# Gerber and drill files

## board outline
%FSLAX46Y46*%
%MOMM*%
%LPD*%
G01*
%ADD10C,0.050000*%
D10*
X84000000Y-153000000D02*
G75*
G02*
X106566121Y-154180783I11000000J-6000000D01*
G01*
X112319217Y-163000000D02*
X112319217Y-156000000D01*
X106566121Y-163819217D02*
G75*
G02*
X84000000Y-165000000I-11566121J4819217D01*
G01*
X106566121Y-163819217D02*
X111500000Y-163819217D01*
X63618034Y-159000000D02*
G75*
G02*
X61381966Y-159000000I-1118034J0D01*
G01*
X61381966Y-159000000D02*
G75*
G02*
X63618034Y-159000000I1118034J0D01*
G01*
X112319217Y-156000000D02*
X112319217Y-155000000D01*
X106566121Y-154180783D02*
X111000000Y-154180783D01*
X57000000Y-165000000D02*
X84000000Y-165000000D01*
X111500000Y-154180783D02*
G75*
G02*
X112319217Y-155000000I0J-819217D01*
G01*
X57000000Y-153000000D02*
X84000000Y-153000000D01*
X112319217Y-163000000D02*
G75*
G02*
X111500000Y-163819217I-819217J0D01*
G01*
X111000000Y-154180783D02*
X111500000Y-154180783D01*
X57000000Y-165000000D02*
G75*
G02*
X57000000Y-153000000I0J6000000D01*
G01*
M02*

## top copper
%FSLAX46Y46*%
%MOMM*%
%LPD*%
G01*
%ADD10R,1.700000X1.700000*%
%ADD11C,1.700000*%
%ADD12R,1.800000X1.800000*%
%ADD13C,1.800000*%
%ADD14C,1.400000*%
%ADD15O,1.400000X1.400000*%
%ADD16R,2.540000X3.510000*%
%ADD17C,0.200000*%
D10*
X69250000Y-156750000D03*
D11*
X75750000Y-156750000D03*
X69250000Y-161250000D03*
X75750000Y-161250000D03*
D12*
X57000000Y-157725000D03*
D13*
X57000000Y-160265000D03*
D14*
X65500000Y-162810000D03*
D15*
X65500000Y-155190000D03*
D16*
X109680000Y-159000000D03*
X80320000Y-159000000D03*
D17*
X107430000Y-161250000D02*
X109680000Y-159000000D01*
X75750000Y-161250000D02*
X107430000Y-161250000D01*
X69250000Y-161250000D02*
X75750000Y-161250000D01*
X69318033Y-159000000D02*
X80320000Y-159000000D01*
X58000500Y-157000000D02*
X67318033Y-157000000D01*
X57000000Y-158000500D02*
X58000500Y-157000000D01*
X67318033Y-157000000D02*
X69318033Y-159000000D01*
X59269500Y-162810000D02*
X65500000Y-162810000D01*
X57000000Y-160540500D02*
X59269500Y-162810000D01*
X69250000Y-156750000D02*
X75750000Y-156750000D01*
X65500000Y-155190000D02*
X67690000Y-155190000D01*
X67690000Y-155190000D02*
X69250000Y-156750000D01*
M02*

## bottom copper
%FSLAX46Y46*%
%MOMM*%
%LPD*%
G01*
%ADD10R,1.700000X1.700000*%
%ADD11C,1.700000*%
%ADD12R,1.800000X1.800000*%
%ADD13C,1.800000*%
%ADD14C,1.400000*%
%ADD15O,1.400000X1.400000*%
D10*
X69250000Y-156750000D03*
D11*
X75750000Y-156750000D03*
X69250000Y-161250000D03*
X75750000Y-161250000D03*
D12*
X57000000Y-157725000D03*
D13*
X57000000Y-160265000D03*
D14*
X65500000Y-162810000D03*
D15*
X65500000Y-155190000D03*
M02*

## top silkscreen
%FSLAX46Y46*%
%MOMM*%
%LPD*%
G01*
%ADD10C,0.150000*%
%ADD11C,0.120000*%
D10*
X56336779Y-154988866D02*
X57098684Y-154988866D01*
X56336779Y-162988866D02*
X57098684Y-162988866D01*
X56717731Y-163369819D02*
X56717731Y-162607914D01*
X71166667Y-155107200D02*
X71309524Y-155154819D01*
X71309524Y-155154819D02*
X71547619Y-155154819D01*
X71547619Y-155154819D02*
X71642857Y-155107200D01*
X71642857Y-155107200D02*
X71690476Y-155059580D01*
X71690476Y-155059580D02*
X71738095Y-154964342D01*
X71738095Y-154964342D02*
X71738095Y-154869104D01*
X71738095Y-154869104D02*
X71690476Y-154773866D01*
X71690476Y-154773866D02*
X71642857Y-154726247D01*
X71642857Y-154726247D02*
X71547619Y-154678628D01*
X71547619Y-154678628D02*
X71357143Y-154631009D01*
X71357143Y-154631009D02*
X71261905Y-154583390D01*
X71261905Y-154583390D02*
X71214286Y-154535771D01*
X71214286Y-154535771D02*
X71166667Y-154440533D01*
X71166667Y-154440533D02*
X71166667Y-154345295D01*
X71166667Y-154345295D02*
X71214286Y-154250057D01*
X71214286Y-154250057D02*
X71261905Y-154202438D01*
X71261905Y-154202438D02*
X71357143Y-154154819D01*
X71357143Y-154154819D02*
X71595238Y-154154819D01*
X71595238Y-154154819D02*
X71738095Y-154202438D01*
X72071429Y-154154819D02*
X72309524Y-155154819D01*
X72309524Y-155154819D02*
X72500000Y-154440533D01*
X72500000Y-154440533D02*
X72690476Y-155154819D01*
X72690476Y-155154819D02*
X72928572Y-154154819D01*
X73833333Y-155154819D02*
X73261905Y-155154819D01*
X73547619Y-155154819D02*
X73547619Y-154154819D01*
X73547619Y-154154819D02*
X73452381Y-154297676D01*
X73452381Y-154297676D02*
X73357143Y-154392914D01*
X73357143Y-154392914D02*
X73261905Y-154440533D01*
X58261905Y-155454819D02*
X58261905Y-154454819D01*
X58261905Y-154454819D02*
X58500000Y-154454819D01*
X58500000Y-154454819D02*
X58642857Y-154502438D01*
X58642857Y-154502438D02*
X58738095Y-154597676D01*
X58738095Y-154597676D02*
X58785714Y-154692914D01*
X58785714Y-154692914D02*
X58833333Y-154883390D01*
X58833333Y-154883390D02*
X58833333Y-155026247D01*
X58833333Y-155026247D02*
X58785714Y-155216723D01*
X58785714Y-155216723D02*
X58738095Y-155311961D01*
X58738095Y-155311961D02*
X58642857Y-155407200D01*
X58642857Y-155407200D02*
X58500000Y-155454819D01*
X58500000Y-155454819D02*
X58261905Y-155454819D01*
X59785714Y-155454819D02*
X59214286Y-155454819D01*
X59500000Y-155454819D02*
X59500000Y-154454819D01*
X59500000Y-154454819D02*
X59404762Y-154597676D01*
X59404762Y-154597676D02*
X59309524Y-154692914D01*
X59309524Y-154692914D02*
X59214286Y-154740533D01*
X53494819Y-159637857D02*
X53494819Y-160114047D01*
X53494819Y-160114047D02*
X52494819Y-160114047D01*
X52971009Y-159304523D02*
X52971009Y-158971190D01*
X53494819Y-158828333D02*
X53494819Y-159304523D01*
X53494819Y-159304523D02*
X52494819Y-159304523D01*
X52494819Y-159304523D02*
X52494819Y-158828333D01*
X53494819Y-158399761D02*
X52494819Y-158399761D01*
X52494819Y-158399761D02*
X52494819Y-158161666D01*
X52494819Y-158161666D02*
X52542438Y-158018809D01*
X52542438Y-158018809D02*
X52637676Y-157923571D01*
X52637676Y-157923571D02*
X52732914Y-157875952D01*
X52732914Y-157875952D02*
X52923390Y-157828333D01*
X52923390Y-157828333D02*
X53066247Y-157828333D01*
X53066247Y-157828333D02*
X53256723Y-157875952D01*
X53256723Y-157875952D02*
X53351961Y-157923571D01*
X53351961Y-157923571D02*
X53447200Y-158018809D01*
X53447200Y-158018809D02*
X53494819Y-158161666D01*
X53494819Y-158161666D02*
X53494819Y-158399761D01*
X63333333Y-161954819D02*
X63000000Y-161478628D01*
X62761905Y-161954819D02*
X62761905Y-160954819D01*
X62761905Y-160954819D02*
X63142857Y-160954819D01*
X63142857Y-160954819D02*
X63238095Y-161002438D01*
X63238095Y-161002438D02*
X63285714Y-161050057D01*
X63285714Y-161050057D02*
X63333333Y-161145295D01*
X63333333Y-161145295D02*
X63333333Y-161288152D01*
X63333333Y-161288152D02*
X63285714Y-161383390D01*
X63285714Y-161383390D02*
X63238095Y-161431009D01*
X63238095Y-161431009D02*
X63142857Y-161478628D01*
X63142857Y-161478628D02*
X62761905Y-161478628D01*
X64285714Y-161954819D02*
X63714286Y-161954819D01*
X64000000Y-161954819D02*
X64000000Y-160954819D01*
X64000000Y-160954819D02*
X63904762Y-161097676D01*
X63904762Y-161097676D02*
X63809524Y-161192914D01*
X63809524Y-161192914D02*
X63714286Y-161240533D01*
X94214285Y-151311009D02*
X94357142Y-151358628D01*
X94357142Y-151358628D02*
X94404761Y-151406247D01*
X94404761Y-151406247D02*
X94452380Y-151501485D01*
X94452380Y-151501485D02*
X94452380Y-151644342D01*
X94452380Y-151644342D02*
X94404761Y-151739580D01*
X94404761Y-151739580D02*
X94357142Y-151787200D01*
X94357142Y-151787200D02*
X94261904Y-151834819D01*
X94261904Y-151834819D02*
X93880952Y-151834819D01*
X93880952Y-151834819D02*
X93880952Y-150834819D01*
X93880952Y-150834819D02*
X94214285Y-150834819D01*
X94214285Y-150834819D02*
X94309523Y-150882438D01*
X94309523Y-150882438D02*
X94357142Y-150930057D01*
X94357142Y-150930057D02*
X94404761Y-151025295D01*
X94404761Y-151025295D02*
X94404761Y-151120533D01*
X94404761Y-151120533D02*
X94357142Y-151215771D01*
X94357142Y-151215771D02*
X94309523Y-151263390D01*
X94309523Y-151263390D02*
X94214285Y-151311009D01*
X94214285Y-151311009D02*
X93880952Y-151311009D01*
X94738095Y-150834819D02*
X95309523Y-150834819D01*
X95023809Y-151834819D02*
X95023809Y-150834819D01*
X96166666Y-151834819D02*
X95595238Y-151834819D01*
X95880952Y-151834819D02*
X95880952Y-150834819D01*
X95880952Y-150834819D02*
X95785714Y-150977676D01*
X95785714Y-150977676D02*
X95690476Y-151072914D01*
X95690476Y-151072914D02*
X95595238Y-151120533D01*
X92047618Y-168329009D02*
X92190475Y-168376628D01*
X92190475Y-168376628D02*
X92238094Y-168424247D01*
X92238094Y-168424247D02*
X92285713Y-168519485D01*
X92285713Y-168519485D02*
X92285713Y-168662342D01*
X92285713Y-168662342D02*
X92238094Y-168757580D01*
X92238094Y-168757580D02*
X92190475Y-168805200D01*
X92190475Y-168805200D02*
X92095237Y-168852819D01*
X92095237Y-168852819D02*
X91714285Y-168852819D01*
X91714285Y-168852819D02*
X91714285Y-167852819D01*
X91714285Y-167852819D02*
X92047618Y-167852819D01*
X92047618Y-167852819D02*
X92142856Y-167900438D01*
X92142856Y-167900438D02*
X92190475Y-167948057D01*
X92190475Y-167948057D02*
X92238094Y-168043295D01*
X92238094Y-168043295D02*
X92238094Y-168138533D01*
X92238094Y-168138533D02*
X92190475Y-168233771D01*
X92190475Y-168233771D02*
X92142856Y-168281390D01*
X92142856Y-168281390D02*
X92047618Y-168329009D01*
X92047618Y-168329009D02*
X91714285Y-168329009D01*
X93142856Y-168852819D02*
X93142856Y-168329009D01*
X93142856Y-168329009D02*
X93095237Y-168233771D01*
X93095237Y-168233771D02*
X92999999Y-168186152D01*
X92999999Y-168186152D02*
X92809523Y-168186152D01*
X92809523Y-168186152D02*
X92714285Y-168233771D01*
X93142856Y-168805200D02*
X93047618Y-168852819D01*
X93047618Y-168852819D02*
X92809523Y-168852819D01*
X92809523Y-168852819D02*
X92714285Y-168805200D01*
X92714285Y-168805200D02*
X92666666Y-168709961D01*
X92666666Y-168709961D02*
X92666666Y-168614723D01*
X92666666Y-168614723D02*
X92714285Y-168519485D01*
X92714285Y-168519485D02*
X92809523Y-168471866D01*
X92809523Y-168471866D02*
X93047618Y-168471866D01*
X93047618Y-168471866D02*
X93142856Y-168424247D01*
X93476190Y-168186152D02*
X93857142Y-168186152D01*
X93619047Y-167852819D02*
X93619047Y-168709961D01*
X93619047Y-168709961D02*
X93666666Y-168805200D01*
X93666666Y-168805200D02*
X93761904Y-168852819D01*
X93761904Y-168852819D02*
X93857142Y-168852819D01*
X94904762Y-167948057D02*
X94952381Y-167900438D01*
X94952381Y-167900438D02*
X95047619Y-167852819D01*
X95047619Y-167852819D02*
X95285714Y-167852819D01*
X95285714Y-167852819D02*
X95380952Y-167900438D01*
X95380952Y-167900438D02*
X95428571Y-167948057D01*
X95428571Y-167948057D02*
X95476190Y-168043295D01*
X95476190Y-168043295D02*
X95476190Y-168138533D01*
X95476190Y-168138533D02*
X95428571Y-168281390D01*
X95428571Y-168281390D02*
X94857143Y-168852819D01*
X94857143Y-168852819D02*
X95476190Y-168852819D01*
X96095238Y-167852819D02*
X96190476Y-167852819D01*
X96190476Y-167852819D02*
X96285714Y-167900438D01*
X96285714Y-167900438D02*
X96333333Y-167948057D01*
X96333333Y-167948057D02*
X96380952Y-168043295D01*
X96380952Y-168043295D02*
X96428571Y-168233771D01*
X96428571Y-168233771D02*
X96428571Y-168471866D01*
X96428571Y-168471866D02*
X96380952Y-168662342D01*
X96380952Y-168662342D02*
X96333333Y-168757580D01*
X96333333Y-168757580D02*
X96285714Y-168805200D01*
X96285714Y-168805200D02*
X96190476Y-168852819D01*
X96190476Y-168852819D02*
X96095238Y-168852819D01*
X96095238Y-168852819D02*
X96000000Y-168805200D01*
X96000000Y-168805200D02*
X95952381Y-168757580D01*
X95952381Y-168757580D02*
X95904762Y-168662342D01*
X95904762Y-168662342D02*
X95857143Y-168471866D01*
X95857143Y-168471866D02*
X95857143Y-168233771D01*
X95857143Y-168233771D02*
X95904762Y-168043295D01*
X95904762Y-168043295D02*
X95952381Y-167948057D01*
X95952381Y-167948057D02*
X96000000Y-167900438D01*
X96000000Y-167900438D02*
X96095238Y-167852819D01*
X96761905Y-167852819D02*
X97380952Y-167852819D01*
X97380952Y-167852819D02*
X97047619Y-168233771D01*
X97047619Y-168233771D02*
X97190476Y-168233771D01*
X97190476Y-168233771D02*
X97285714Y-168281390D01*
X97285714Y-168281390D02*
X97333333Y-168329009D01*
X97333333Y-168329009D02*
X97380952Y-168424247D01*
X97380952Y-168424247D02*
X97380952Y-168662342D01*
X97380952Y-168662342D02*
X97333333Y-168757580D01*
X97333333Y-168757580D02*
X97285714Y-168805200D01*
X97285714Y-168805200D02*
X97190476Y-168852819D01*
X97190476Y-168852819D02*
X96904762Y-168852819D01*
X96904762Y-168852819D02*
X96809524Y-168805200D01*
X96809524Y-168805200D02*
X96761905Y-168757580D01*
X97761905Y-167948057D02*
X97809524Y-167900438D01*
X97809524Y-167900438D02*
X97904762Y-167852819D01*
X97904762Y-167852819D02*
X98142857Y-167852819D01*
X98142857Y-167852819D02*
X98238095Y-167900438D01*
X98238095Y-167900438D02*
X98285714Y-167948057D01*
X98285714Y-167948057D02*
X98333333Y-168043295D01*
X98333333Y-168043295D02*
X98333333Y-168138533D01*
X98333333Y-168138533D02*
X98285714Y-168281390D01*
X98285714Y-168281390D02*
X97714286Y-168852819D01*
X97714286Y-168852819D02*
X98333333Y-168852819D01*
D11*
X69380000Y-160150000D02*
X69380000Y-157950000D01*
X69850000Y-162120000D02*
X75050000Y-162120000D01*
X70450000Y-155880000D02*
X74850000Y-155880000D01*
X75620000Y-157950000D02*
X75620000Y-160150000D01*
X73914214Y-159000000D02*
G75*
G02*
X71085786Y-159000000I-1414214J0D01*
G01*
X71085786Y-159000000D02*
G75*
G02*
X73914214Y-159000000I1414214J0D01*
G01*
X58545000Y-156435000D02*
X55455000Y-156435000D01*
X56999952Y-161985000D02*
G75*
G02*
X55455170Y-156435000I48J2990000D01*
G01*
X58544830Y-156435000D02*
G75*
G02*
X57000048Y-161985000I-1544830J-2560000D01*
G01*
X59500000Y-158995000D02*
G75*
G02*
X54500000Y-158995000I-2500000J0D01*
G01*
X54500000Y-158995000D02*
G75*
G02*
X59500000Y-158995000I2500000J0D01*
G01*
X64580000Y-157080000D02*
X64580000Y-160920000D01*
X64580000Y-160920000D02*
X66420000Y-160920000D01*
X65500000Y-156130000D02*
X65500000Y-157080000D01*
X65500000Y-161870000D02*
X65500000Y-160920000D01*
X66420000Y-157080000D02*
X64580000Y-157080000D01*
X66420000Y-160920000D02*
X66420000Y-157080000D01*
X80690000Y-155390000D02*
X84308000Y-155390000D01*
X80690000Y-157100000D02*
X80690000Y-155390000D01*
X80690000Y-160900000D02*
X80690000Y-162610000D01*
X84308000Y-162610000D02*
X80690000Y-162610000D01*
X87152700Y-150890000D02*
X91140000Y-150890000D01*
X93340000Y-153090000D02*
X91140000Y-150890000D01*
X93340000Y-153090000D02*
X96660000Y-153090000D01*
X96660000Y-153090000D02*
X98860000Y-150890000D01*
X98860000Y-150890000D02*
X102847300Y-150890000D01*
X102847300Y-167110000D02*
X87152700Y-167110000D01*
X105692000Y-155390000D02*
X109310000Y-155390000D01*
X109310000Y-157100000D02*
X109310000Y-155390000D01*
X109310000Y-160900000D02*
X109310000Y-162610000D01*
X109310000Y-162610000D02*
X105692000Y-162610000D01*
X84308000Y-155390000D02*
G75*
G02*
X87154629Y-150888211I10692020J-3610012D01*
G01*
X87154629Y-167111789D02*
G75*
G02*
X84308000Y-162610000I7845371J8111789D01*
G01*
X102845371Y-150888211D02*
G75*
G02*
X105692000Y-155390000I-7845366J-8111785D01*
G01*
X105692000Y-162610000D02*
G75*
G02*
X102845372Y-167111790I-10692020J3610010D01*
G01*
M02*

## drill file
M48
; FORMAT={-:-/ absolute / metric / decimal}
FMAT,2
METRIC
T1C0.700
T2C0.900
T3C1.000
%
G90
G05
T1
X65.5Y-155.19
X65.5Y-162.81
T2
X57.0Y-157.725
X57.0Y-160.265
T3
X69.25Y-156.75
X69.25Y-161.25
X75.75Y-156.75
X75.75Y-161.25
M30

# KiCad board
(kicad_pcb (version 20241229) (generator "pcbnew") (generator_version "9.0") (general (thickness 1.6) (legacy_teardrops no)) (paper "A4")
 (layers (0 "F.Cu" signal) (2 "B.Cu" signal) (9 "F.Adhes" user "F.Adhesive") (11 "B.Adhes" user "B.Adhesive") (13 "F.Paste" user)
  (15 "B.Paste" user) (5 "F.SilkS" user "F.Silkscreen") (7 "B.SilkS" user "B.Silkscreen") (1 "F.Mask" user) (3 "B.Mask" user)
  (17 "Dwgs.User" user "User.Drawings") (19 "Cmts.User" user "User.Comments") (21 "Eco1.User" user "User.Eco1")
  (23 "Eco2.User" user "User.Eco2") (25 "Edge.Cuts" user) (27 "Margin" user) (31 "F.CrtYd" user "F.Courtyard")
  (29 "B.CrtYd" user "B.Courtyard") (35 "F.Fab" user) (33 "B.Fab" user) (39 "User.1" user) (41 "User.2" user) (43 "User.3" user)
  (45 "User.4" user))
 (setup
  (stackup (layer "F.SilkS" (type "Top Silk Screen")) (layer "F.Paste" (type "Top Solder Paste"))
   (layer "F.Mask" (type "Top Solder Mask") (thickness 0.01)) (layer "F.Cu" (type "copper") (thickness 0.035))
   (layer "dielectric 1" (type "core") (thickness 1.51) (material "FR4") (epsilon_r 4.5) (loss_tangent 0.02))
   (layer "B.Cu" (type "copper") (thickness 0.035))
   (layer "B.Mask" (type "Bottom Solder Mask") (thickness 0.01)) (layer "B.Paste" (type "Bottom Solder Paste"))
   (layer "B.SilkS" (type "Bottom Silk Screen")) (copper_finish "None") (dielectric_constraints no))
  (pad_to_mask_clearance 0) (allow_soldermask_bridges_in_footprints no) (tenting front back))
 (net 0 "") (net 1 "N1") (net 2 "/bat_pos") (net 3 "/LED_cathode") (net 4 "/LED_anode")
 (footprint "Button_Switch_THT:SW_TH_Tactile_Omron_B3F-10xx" (layer "F.Cu") (at 69.25 156.75)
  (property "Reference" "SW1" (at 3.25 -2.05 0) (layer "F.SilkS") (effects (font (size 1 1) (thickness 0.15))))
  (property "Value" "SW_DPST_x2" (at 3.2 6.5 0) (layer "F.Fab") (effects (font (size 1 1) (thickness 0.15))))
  (fp_line (start 0.13 3.4) (end 0.13 1.2) (stroke (width 0.12) (type solid)) (layer "F.SilkS"))
  (fp_line (start 0.6 5.37) (end 5.8 5.37) (stroke (width 0.12) (type solid)) (layer "F.SilkS"))
  (fp_line (start 1.2 -0.87) (end 5.6 -0.87) (stroke (width 0.12) (type solid)) (layer "F.SilkS"))
  (fp_line (start 6.37 1.2) (end 6.37 3.4) (stroke (width 0.12) (type solid)) (layer "F.SilkS"))
  (fp_circle (center 3.25 2.25) (end 4.25 3.25) (stroke (width 0.12) (type solid)) (fill no) (layer "F.SilkS"))
  (pad "1" thru_hole rect (at 0 0) (size 1.7 1.7) (drill 1) (layers "*.Cu" "*.Mask") (remove_unused_layers no) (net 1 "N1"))
  (pad "1" thru_hole circle (at 6.5 0) (size 1.7 1.7) (drill 1) (layers "*.Cu" "*.Mask") (remove_unused_layers no) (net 1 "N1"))
  (pad "2" thru_hole circle (at 0 4.5) (size 1.7 1.7) (drill 1) (layers "*.Cu" "*.Mask") (remove_unused_layers no) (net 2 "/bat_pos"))
  (pad "2" thru_hole circle (at 6.5 4.5) (size 1.7 1.7) (drill 1) (layers "*.Cu" "*.Mask") (remove_unused_layers no) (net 2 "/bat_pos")))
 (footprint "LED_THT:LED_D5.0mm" (layer "F.Cu") (at 57 157.725 -90)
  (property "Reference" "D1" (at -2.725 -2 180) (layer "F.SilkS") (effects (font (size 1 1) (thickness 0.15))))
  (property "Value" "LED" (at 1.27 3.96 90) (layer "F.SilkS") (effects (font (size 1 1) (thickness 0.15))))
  (fp_line (start -1.29 -1.545) (end -1.29 1.545) (stroke (width 0.12) (type solid)) (layer "F.SilkS"))
  (fp_arc (start 4.26 0.000048) (mid 2.071756 2.880501) (end -1.29 1.54483) (stroke (width 0.12) (type solid)) (layer "F.SilkS"))
  (fp_arc (start -1.29 -1.54483) (mid 2.071756 -2.880501) (end 4.26 -0.000048) (stroke (width 0.12) (type solid)) (layer "F.SilkS"))
  (fp_circle (center 1.27 0) (end 3.77 0) (stroke (width 0.12) (type solid)) (fill no) (layer "F.SilkS"))
  (pad "1" thru_hole rect (at 0 0 270) (size 1.8 1.8) (drill 0.9) (layers "*.Cu" "*.Mask") (remove_unused_layers no) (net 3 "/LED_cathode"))
  (pad "2" thru_hole circle (at 2.54 0 270) (size 1.8 1.8) (drill 0.9) (layers "*.Cu" "*.Mask") (remove_unused_layers no)
   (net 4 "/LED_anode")))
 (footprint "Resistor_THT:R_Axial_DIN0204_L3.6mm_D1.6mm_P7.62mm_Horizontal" (layer "F.Cu") (at 65.5 162.81 90)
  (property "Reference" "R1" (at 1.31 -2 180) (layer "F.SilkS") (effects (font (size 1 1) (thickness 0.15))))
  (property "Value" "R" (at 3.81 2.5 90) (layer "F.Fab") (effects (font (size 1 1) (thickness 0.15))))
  (fp_line (start 5.73 -0.92) (end 1.89 -0.92) (stroke (width 0.12) (type solid)) (layer "F.SilkS"))
  (fp_line (start 1.89 -0.92) (end 1.89 0.92) (stroke (width 0.12) (type solid)) (layer "F.SilkS"))
  (fp_line (start 6.68 0) (end 5.73 0) (stroke (width 0.12) (type solid)) (layer "F.SilkS"))
  (fp_line (start 0.94 0) (end 1.89 0) (stroke (width 0.12) (type solid)) (layer "F.SilkS"))
  (fp_line (start 5.73 0.92) (end 5.73 -0.92) (stroke (width 0.12) (type solid)) (layer "F.SilkS"))
  (fp_line (start 1.89 0.92) (end 5.73 0.92) (stroke (width 0.12) (type solid)) (layer "F.SilkS"))
  (pad "1" thru_hole circle (at 0 0 90) (size 1.4 1.4) (drill 0.7) (layers "*.Cu" "*.Mask") (remove_unused_layers no) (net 4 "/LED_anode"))
  (pad "2" thru_hole oval (at 7.62 0 90) (size 1.4 1.4) (drill 0.7) (layers "*.Cu" "*.Mask") (remove_unused_layers no) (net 1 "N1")))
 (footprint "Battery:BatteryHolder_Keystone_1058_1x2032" (layer "F.Cu") (at 95 159 180)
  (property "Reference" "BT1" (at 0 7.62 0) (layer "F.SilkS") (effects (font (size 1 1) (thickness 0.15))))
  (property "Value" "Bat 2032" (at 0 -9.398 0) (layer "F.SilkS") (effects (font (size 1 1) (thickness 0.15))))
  (fp_line (start 14.31 3.61) (end 10.692 3.61) (stroke (width 0.12) (type solid)) (layer "F.SilkS"))
  (fp_line (start 14.31 1.9) (end 14.31 3.61) (stroke (width 0.12) (type solid)) (layer "F.SilkS"))
  (fp_line (start 14.31 -1.9) (end 14.31 -3.61) (stroke (width 0.12) (type solid)) (layer "F.SilkS"))
  (fp_line (start 10.692 -3.61) (end 14.31 -3.61) (stroke (width 0.12) (type solid)) (layer "F.SilkS"))
  (fp_line (start 7.8473 8.11) (end 3.86 8.11) (stroke (width 0.12) (type solid)) (layer "F.SilkS"))
  (fp_line (start 1.66 5.91) (end 3.86 8.11) (stroke (width 0.12) (type solid)) (layer "F.SilkS"))
  (fp_line (start 1.66 5.91) (end -1.66 5.91) (stroke (width 0.12) (type solid)) (layer "F.SilkS"))
  (fp_line (start -1.66 5.91) (end -3.86 8.11) (stroke (width 0.12) (type solid)) (layer "F.SilkS"))
  (fp_line (start -3.86 8.11) (end -7.8473 8.11) (stroke (width 0.12) (type solid)) (layer "F.SilkS"))
  (fp_line (start -7.8473 -8.11) (end 7.8473 -8.11) (stroke (width 0.12) (type solid)) (layer "F.SilkS"))
  (fp_line (start -10.692 3.61) (end -14.31 3.61) (stroke (width 0.12) (type solid)) (layer "F.SilkS"))
  (fp_line (start -14.31 1.9) (end -14.31 3.61) (stroke (width 0.12) (type solid)) (layer "F.SilkS"))
  (fp_line (start -14.31 -1.9) (end -14.31 -3.61) (stroke (width 0.12) (type solid)) (layer "F.SilkS"))
  (fp_line (start -14.31 -3.61) (end -10.692 -3.61) (stroke (width 0.12) (type solid)) (layer "F.SilkS"))
  (fp_arc (start 10.692 3.61) (mid 9.538084 6.031244) (end 7.845371 8.111789) (stroke (width 0.12) (type solid)) (layer "F.SilkS"))
  (fp_arc (start 7.845371 -8.111789) (mid 9.538085 -6.031244) (end 10.692 -3.61) (stroke (width 0.12) (type solid)) (layer "F.SilkS"))
  (fp_arc (start -7.845371 8.111789) (mid -9.538085 6.031244) (end -10.692 3.61) (stroke (width 0.12) (type solid)) (layer "F.SilkS"))
  (fp_arc (start -10.692 -3.61) (mid -9.538084 -6.031244) (end -7.845371 -8.111789) (stroke (width 0.12) (type solid)) (layer "F.SilkS"))
  (pad "1" smd rect (at -14.68 0 180) (size 2.54 3.51) (layers "F.Cu" "F.Mask" "F.Paste") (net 2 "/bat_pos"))
  (pad "2" smd rect (at 14.68 0 180) (size 2.54 3.51) (layers "F.Cu" "F.Mask" "F.Paste") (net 3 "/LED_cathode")))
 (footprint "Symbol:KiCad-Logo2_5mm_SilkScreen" (layer "B.Cu") (at 96 156.5 180)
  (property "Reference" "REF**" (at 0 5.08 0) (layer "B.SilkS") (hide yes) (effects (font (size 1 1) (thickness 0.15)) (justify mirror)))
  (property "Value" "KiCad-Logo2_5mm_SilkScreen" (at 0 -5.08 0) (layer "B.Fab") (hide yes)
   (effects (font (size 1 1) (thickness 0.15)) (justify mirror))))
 (gr_arc (start 84 153) (mid 95.654741 146.487154) (end 106.566121 154.180783) (stroke (width 0.05) (type default)) (locked yes)
  (layer "Edge.Cuts"))
 (gr_line (start 112.319217 163) (end 112.319217 156) (stroke (width 0.05) (type default)) (locked yes) (layer "Edge.Cuts"))
 (gr_arc (start 106.566121 163.819217) (mid 95.654741 171.512846) (end 84 165) (stroke (width 0.05) (type default)) (locked yes)
  (layer "Edge.Cuts"))
 (gr_line (start 106.566121 163.819217) (end 111.5 163.819217) (stroke (width 0.05) (type default)) (locked yes) (layer "Edge.Cuts"))
 (gr_circle (center 62.5 159) (end 63 160) (stroke (width 0.05) (type default)) (fill no) (layer "Edge.Cuts"))
 (gr_line (start 112.319217 156) (end 112.319217 155) (stroke (width 0.05) (type default)) (locked yes) (layer "Edge.Cuts"))
 (gr_line (start 106.566121 154.180783) (end 111 154.180783) (stroke (width 0.05) (type default)) (locked yes) (layer "Edge.Cuts"))
 (gr_line (start 57 165) (end 84 165) (stroke (width 0.05) (type default)) (locked yes) (layer "Edge.Cuts"))
 (gr_arc (start 111.5 154.180783) (mid 112.079274 154.420726) (end 112.319217 155) (stroke (width 0.05) (type default)) (locked yes)
  (layer "Edge.Cuts"))
 (gr_line (start 57 153) (end 84 153) (stroke (width 0.05) (type default)) (locked yes) (layer "Edge.Cuts"))
 (gr_arc (start 112.319217 163) (mid 112.079274 163.579274) (end 111.5 163.819217) (stroke (width 0.05) (type default)) (locked yes)
  (layer "Edge.Cuts"))
 (gr_line (start 111 154.180783) (end 111.5 154.180783) (stroke (width 0.05) (type default)) (locked yes) (layer "Edge.Cuts"))
 (gr_arc (start 57 165) (mid 51 159) (end 57 153) (stroke (width 0.05) (type default)) (locked yes) (layer "Edge.Cuts"))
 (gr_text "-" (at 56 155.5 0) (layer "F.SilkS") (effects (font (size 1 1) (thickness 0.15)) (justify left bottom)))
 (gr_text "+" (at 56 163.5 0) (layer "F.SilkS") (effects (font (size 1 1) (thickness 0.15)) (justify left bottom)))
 (segment (start 107.43 161.25) (end 109.68 159) (width 0.2) (layer "F.Cu") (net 2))
 (segment (start 75.75 161.25) (end 107.43 161.25) (width 0.2) (layer "F.Cu") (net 2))
 (segment (start 69.25 161.25) (end 75.75 161.25) (width 0.2) (layer "F.Cu") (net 2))
 (segment (start 69.318033 159) (end 80.32 159) (width 0.2) (layer "F.Cu") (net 3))
 (segment (start 58.0005 157) (end 67.318033 157) (width 0.2) (layer "F.Cu") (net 3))
 (segment (start 57 158.0005) (end 58.0005 157) (width 0.2) (layer "F.Cu") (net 3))
 (segment (start 67.318033 157) (end 69.318033 159) (width 0.2) (layer "F.Cu") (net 3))
 (segment (start 59.2695 162.81) (end 65.5 162.81) (width 0.2) (layer "F.Cu") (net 4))
 (segment (start 57 160.5405) (end 59.2695 162.81) (width 0.2) (layer "F.Cu") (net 4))
 (segment (start 69.25 156.75) (end 75.75 156.75) (width 0.2) (layer "F.Cu") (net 1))
 (segment (start 65.5 155.19) (end 67.69 155.19) (width 0.2) (layer "F.Cu") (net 1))
 (segment (start 67.69 155.19) (end 69.25 156.75) (width 0.2) (layer "F.Cu") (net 1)))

